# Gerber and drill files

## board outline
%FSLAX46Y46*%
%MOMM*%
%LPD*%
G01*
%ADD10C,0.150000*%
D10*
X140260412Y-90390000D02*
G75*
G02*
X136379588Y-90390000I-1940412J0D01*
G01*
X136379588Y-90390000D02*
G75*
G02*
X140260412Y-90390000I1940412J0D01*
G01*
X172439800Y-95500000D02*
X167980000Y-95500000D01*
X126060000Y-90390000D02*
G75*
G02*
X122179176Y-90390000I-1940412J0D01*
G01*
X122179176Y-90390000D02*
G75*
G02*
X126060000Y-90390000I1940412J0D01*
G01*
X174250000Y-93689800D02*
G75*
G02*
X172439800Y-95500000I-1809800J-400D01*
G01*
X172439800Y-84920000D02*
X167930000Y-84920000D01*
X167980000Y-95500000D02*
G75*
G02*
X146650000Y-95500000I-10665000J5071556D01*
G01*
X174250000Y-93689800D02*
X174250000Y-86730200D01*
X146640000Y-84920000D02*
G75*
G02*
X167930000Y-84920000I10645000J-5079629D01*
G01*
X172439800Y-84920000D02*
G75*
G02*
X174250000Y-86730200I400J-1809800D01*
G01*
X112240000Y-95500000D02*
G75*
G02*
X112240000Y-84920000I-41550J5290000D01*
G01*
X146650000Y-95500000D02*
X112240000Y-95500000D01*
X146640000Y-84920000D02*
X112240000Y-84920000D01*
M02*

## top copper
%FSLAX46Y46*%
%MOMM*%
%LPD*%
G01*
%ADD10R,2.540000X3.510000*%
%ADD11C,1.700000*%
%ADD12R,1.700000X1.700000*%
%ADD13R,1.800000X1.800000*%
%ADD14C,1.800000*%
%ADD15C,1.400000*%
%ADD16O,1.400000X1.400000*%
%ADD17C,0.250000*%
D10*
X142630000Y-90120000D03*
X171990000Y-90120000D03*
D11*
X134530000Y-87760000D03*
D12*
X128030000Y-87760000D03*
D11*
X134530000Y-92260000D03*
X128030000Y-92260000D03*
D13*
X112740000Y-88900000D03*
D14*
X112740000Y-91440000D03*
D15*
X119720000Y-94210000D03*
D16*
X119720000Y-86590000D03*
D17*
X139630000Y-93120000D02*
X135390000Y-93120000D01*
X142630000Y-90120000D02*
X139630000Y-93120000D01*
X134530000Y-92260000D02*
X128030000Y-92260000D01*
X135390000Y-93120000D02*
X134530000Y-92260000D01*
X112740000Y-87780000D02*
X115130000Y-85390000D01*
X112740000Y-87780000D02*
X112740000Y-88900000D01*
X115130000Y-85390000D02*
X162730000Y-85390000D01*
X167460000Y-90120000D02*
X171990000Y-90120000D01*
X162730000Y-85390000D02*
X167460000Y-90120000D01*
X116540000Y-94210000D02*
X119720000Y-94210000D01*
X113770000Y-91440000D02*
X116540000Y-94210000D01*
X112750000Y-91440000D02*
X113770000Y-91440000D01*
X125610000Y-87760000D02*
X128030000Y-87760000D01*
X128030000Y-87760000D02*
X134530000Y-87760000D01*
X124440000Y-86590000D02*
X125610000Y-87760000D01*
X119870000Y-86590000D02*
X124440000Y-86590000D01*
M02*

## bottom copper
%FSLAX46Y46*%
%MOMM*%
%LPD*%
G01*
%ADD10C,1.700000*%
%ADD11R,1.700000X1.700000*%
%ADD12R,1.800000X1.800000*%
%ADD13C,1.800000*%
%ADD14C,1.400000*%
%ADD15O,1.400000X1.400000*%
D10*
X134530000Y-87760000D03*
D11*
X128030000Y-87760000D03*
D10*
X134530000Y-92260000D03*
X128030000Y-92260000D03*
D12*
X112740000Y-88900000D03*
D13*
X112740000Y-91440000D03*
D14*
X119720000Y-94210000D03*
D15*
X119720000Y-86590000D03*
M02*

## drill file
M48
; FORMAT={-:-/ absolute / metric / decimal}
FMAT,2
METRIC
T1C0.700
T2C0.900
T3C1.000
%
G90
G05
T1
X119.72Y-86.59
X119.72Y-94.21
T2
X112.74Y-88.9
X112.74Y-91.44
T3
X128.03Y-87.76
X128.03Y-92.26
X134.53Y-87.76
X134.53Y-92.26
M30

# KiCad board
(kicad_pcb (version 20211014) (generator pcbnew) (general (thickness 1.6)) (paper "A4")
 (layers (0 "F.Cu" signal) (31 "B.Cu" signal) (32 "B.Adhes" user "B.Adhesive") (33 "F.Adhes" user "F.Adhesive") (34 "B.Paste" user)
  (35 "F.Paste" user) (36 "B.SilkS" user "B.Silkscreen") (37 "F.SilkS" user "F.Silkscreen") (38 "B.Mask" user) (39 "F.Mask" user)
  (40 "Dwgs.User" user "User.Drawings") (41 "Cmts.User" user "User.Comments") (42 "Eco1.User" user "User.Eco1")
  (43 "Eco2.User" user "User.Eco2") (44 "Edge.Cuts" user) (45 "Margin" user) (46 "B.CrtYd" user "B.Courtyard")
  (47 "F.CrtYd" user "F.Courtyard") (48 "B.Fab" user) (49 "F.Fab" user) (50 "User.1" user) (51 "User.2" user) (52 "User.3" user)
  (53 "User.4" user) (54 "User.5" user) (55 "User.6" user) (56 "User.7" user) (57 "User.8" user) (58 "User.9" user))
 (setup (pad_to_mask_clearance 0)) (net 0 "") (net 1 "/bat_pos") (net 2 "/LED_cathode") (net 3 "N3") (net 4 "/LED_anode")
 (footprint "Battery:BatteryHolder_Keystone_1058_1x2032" (layer "F.Cu") (at 157.31 90.12)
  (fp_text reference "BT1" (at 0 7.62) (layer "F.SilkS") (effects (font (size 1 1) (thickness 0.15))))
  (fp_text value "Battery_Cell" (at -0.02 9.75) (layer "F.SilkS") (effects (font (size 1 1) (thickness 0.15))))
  (pad "1" smd rect (at -14.68 0) (size 2.54 3.51) (layers "F.Cu" "F.Paste" "F.Mask") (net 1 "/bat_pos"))
  (pad "2" smd rect (at 14.68 0) (size 2.54 3.51) (layers "F.Cu" "F.Paste" "F.Mask") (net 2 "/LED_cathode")))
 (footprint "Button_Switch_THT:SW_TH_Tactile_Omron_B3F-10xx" (layer "F.Cu") (at 128.03 87.76)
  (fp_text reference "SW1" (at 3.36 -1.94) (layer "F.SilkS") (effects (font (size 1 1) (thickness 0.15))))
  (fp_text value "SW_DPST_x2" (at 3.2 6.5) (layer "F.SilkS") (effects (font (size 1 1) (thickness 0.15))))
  (pad "1" thru_hole circle (at 6.5 0) (size 1.7 1.7) (drill 1) (layers *.Cu *.Mask) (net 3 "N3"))
  (pad "1" thru_hole rect (at 0 0) (size 1.7 1.7) (drill 1) (layers *.Cu *.Mask) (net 3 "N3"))
  (pad "2" thru_hole circle (at 6.5 4.5) (size 1.7 1.7) (drill 1) (layers *.Cu *.Mask) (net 1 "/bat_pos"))
  (pad "2" thru_hole circle (at 0 4.5) (size 1.7 1.7) (drill 1) (layers *.Cu *.Mask) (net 1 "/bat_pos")))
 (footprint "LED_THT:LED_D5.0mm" (layer "F.Cu") (at 112.74 88.9 -90)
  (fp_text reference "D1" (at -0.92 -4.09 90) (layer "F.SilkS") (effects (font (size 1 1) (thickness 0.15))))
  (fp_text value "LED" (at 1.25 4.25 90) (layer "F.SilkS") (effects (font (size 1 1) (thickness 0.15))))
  (pad "1" thru_hole rect (at 0 0 270) (size 1.8 1.8) (drill 0.9) (layers *.Cu *.Mask) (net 2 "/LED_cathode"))
  (pad "2" thru_hole circle (at 2.54 0 270) (size 1.8 1.8) (drill 0.9) (layers *.Cu *.Mask) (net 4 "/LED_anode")))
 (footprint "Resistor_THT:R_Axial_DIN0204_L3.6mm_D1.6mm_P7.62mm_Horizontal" (layer "F.Cu") (at 119.72 94.21 90)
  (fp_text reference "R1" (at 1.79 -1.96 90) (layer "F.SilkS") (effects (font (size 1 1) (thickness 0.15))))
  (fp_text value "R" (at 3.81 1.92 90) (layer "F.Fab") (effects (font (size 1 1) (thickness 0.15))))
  (pad "1" thru_hole circle (at 0 0 90) (size 1.4 1.4) (drill 0.7) (layers *.Cu *.Mask) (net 4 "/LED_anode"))
  (pad "2" thru_hole oval (at 7.62 0 90) (size 1.4 1.4) (drill 0.7) (layers *.Cu *.Mask) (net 3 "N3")))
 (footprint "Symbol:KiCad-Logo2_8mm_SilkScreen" (layer "B.Cu") (at 157.18 88.95 180)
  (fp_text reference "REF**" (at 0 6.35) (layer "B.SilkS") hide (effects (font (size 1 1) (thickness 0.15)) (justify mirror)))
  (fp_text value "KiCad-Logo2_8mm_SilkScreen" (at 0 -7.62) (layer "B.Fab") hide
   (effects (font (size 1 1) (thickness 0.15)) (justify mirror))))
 (gr_circle (center 138.32 90.39) (end 140.260412 90.39) (layer "Edge.Cuts") (width 0.15) (fill none))
 (gr_line (start 172.4398 95.5) (end 167.98 95.5) (layer "Edge.Cuts") (width 0.15))
 (gr_circle (center 124.119588 90.39) (end 126.06 90.39) (layer "Edge.Cuts") (width 0.15) (fill none))
 (gr_arc (start 174.25 93.6898) (mid 173.719917 94.969917) (end 172.4398 95.5) (layer "Edge.Cuts") (width 0.15))
 (gr_line (start 172.4398 84.92) (end 167.93 84.92) (layer "Edge.Cuts") (width 0.15))
 (gr_arc (start 167.98 95.5) (mid 157.312447 102.237885) (end 146.65 95.5) (layer "Edge.Cuts") (width 0.15))
 (gr_line (start 174.25 93.6898) (end 174.25 86.7302) (layer "Edge.Cuts") (width 0.15))
 (gr_arc (start 146.64 84.92) (mid 157.284081 78.204772) (end 167.93 84.92) (layer "Edge.Cuts") (width 0.15))
 (gr_arc (start 172.4398 84.92) (mid 173.719921 85.450079) (end 174.25 86.7302) (layer "Edge.Cuts") (width 0.15))
 (gr_arc (start 112.24 95.5) (mid 106.908289 90.21) (end 112.24 84.92) (layer "Edge.Cuts") (width 0.15))
 (gr_line (start 146.65 95.5) (end 112.24 95.5) (layer "Edge.Cuts") (width 0.15))
 (gr_line (start 146.64 84.92) (end 112.24 84.92) (layer "Edge.Cuts") (width 0.15))
 (segment (start 139.63 93.12) (end 135.39 93.12) (width 0.25) (layer "F.Cu") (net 1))
 (segment (start 142.63 90.12) (end 139.63 93.12) (width 0.25) (layer "F.Cu") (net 1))
 (segment (start 134.53 92.26) (end 128.03 92.26) (width 0.25) (layer "F.Cu") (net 1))
 (segment (start 135.39 93.12) (end 134.53 92.26) (width 0.25) (layer "F.Cu") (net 1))
 (segment (start 112.74 87.78) (end 115.13 85.39) (width 0.25) (layer "F.Cu") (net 2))
 (segment (start 112.74 87.78) (end 112.74 88.9) (width 0.25) (layer "F.Cu") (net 2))
 (segment (start 115.13 85.39) (end 162.73 85.39) (width 0.25) (layer "F.Cu") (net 2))
 (segment (start 167.46 90.12) (end 171.99 90.12) (width 0.25) (layer "F.Cu") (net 2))
 (segment (start 162.73 85.39) (end 167.46 90.12) (width 0.25) (layer "F.Cu") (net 2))
 (segment (start 116.54 94.21) (end 119.72 94.21) (width 0.25) (layer "F.Cu") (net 4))
 (segment (start 113.77 91.44) (end 116.54 94.21) (width 0.25) (layer "F.Cu") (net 4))
 (segment (start 112.75 91.44) (end 113.77 91.44) (width 0.25) (layer "F.Cu") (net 4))
 (segment (start 125.61 87.76) (end 128.03 87.76) (width 0.25) (layer "F.Cu") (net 3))
 (segment (start 128.03 87.76) (end 134.53 87.76) (width 0.25) (layer "F.Cu") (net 3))
 (segment (start 124.44 86.59) (end 125.61 87.76) (width 0.25) (layer "F.Cu") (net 3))
 (segment (start 119.87 86.59) (end 124.44 86.59) (width 0.25) (layer "F.Cu") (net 3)))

